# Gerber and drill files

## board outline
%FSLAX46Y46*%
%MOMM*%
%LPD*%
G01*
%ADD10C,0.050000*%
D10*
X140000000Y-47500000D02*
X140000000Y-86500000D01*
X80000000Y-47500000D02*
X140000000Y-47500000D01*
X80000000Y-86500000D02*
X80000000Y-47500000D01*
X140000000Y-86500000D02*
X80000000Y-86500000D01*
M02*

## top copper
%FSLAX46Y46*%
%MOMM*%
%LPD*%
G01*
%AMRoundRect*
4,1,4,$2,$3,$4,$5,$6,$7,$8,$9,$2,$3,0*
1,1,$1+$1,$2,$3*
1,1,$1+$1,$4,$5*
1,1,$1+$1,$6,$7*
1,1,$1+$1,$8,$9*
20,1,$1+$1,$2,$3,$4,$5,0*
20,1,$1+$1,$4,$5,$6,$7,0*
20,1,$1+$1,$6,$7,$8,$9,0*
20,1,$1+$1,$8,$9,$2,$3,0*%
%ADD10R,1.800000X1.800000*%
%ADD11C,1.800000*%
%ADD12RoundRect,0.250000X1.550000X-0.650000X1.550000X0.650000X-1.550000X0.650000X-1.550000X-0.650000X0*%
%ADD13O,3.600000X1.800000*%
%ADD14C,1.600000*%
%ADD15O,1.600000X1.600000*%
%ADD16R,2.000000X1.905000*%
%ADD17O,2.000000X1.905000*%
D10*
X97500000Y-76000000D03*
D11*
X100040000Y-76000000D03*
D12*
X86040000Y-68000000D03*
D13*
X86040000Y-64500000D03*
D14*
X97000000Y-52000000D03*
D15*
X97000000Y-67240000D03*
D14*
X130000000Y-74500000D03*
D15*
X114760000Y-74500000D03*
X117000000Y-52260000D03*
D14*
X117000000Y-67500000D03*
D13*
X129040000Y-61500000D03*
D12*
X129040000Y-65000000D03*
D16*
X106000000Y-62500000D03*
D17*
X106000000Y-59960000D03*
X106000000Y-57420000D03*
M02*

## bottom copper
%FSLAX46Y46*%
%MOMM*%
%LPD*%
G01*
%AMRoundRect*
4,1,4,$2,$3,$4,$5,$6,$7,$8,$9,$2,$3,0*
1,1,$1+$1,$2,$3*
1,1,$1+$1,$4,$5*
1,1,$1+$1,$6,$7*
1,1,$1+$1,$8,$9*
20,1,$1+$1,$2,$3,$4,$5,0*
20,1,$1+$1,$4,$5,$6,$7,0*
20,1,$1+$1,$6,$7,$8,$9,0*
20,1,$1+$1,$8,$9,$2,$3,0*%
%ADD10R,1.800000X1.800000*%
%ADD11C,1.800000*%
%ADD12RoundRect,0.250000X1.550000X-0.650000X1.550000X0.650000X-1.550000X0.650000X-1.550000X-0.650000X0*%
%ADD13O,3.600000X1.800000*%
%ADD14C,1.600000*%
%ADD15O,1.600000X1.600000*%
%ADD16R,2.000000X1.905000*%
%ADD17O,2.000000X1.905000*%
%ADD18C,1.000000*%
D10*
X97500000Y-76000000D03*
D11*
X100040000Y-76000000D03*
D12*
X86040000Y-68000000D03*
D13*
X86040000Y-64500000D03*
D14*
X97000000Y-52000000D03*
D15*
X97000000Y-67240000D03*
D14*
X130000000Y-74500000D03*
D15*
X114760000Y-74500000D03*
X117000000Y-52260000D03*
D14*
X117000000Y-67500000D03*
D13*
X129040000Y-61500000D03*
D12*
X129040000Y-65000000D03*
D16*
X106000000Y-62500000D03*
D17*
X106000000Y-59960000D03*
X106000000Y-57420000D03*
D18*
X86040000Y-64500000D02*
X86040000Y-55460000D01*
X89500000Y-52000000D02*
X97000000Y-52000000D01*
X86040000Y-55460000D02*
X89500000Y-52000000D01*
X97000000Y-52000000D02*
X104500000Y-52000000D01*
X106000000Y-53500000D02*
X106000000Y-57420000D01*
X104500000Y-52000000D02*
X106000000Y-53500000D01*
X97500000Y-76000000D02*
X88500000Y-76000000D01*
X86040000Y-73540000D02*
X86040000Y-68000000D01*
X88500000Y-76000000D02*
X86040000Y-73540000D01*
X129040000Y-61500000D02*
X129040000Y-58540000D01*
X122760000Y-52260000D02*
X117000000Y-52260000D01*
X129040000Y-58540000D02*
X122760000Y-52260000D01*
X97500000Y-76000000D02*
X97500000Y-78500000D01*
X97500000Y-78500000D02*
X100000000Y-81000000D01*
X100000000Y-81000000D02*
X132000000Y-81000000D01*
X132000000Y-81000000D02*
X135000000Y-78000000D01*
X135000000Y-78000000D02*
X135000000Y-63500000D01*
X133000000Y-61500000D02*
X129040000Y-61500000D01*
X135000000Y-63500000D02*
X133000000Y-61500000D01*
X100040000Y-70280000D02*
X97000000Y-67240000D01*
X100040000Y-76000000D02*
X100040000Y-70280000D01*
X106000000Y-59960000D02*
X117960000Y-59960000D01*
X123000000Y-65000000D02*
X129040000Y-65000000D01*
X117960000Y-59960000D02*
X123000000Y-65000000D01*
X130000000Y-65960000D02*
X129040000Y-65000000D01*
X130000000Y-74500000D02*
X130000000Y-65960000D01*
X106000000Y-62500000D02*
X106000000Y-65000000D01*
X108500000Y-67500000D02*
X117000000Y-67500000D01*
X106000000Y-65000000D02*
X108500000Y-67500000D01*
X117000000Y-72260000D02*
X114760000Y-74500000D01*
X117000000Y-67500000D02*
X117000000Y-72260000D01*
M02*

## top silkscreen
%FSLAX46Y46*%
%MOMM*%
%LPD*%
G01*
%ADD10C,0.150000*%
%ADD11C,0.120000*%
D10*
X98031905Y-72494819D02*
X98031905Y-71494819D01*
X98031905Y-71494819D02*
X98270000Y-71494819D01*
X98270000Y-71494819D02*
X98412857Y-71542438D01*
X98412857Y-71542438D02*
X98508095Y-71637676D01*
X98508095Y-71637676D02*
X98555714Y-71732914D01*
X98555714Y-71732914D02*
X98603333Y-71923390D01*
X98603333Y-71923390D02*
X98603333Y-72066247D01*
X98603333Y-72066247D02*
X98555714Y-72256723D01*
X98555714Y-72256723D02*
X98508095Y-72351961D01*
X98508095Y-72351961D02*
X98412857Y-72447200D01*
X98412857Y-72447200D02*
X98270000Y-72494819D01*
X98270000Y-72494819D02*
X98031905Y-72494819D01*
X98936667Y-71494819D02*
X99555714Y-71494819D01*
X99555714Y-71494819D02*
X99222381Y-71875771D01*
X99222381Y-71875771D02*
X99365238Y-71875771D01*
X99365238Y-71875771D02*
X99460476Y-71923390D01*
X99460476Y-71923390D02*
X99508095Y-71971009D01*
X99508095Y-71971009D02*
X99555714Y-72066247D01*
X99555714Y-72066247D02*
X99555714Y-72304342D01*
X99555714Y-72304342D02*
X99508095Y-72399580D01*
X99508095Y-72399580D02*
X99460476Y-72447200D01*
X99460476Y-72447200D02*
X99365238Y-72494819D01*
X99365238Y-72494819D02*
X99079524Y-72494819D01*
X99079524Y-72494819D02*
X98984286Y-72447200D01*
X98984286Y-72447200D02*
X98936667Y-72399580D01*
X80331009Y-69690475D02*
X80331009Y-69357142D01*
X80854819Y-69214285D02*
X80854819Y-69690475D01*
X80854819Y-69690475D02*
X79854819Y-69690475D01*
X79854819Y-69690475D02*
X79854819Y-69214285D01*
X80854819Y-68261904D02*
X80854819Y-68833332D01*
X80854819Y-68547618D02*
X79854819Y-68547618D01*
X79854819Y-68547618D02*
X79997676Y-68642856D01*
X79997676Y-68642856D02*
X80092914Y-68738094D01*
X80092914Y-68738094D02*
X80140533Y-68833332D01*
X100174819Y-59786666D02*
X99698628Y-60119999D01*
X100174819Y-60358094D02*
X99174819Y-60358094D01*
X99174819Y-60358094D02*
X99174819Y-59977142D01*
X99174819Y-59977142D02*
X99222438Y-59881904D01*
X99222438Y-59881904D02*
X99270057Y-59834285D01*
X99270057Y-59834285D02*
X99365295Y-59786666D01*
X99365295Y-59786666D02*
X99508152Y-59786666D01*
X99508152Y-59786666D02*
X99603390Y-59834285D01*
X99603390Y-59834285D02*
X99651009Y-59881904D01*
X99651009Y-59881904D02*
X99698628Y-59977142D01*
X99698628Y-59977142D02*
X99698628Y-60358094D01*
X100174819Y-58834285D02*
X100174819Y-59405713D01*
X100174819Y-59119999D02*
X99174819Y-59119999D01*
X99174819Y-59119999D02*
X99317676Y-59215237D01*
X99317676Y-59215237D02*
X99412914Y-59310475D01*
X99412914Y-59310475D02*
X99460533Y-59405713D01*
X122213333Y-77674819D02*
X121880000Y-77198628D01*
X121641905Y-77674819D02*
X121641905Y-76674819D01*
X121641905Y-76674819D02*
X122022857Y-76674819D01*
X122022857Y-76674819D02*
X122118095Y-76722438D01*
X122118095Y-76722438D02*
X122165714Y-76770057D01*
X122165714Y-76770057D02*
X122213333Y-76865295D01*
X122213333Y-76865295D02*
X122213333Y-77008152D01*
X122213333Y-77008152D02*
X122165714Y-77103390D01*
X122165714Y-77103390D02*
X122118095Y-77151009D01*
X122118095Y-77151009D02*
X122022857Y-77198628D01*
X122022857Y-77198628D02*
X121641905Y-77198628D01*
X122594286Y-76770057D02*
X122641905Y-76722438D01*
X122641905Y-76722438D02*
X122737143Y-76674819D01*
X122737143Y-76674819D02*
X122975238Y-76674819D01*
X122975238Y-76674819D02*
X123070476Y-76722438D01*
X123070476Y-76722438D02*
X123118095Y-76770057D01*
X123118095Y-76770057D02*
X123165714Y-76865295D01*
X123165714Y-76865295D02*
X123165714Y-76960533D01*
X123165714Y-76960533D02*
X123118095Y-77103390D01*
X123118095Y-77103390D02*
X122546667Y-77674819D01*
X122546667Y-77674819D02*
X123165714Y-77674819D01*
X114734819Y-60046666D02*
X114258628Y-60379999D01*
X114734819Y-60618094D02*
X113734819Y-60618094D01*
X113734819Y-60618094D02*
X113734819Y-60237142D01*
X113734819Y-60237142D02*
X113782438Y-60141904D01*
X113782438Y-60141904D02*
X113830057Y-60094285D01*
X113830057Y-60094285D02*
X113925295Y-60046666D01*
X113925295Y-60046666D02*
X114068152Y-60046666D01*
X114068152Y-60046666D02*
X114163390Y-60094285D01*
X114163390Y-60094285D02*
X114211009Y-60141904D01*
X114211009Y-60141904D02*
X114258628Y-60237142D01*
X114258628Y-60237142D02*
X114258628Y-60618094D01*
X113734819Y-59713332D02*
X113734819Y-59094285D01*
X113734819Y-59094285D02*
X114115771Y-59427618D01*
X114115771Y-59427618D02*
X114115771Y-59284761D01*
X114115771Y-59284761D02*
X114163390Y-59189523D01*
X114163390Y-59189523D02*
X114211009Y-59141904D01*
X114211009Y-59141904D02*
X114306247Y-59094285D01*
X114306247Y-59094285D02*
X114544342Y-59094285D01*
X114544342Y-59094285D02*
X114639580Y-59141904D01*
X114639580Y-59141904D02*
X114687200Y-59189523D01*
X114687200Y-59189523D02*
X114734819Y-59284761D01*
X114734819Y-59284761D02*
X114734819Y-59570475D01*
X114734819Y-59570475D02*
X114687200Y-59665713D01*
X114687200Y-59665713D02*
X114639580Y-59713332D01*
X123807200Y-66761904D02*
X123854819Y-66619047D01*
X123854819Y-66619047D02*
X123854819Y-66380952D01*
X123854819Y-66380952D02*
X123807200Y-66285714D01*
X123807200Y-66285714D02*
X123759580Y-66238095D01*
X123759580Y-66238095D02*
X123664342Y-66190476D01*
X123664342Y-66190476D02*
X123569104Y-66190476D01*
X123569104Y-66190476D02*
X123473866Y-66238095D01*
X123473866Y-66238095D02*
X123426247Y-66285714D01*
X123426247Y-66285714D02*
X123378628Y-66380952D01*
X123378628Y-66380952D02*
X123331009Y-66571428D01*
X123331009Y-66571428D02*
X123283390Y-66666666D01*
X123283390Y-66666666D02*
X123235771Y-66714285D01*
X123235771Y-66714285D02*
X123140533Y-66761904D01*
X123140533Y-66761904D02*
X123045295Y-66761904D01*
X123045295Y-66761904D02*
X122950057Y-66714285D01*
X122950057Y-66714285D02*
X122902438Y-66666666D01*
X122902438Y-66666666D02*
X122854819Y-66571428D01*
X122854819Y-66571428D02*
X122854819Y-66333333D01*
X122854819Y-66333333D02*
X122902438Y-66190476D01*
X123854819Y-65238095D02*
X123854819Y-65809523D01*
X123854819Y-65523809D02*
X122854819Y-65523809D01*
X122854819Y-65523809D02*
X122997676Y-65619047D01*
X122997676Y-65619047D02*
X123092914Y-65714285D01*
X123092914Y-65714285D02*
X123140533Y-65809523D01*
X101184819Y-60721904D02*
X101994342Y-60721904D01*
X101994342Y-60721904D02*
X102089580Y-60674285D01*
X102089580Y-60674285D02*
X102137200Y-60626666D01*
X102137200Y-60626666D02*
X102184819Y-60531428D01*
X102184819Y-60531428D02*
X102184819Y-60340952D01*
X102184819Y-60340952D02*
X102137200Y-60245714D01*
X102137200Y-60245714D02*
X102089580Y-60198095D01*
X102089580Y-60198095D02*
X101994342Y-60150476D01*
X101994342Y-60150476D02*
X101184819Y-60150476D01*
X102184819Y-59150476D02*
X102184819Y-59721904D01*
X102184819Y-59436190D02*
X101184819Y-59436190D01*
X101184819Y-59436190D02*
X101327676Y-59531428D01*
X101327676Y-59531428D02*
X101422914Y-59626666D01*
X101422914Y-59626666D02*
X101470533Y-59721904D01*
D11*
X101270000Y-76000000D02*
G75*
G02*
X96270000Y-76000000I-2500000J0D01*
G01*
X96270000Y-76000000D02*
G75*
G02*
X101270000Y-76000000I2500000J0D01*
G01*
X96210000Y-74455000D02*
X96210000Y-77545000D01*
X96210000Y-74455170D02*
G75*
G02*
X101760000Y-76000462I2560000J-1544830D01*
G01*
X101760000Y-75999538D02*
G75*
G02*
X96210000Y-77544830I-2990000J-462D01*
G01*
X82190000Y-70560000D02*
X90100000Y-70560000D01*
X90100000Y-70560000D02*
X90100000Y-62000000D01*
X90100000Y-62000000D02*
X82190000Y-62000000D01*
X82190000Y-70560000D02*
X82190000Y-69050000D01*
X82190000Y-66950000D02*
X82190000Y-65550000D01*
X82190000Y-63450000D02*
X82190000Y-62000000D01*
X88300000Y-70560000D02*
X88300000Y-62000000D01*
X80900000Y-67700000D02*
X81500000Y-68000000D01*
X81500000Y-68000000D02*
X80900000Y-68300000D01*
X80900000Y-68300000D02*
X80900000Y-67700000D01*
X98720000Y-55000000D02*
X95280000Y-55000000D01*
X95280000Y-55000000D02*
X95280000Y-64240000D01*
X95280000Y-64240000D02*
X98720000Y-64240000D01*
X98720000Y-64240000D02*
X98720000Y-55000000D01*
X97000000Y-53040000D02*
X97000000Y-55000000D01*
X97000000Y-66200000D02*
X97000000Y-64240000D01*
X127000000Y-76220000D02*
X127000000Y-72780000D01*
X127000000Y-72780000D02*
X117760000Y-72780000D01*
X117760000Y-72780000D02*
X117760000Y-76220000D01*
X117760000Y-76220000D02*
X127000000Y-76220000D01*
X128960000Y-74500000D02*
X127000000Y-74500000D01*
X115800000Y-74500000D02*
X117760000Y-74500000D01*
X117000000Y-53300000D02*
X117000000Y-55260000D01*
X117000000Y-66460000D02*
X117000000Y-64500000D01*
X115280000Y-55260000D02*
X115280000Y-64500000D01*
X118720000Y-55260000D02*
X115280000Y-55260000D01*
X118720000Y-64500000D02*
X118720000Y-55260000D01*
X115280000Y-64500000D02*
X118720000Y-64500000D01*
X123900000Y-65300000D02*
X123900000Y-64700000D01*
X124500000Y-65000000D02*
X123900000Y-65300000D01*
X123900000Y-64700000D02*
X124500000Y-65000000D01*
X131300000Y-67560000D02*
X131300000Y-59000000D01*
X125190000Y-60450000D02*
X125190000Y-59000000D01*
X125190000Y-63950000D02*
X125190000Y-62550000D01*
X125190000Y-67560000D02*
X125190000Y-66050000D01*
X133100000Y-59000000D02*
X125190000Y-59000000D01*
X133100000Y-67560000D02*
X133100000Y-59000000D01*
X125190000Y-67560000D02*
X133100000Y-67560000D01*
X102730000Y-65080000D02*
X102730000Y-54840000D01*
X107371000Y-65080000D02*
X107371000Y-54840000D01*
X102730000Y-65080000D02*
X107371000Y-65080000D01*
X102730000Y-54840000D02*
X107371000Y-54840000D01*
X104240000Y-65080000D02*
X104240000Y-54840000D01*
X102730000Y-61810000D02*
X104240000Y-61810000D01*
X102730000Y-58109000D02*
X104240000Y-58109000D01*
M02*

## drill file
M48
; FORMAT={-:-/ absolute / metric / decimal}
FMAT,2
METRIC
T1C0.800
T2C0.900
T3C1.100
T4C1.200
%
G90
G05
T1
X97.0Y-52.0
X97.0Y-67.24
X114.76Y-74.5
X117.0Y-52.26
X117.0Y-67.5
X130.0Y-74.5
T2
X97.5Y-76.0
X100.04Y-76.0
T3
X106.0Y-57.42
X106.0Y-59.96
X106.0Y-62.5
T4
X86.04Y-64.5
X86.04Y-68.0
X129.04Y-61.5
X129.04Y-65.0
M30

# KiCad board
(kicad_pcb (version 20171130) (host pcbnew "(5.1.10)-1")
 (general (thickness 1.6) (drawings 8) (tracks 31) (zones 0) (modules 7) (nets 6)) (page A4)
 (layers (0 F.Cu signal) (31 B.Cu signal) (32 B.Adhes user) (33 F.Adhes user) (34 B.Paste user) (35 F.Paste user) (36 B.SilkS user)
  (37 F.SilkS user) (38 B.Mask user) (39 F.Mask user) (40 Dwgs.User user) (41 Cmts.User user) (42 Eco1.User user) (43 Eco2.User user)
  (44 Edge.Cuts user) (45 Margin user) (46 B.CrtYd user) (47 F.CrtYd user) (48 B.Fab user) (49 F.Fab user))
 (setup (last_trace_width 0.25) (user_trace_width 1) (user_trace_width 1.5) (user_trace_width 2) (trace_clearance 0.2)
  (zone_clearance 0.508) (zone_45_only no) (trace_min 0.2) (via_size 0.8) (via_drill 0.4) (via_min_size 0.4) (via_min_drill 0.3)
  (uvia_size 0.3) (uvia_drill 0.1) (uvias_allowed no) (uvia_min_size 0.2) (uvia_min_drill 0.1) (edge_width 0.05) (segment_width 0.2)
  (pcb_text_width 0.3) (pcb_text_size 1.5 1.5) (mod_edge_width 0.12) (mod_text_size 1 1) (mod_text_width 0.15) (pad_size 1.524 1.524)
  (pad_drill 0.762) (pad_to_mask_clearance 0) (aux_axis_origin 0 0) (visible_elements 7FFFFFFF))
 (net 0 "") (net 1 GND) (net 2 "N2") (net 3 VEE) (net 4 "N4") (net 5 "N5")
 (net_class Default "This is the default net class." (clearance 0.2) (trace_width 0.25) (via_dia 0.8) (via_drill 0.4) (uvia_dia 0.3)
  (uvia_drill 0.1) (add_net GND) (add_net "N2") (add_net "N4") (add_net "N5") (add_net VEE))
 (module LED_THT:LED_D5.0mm (layer F.Cu) (at 97.5 76)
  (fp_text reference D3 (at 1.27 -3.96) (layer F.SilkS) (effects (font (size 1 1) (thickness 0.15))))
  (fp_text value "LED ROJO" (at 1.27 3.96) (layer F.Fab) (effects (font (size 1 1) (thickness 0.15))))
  (fp_circle (center 1.27 0) (end 3.77 0) (layer F.SilkS) (width 0.12))
  (fp_line (start -1.29 -1.545) (end -1.29 1.545) (layer F.SilkS) (width 0.12))
  (fp_arc (start 1.27 0) (end -1.29 -1.54483) (angle 148.9) (layer F.SilkS) (width 0.12))
  (fp_arc (start 1.27 0) (end -1.29 1.54483) (angle -148.9) (layer F.SilkS) (width 0.12))
  (pad 1 thru_hole rect (at 0 0) (size 1.8 1.8) (drill 0.9) (layers *.Cu *.Mask) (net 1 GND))
  (pad 2 thru_hole circle (at 2.54 0) (size 1.8 1.8) (drill 0.9) (layers *.Cu *.Mask) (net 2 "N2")))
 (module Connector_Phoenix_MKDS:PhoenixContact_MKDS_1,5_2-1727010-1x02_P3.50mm (layer F.Cu) (at 83.5 68 90)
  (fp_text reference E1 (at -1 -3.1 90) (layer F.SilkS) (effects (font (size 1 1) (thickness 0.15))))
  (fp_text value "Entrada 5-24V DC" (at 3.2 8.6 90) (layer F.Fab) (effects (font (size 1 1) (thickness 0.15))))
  (fp_line (start -2.56 -1.31) (end -2.56 6.6) (layer F.SilkS) (width 0.12))
  (fp_line (start -2.56 6.6) (end 6 6.6) (layer F.SilkS) (width 0.12))
  (fp_line (start 6 6.6) (end 6 -1.31) (layer F.SilkS) (width 0.12))
  (fp_line (start -2.56 -1.31) (end -1.05 -1.31) (layer F.SilkS) (width 0.12))
  (fp_line (start 1.05 -1.31) (end 2.45 -1.31) (layer F.SilkS) (width 0.12))
  (fp_line (start 4.55 -1.31) (end 6 -1.31) (layer F.SilkS) (width 0.12))
  (fp_line (start -2.56 4.8) (end 6 4.8) (layer F.SilkS) (width 0.12))
  (fp_line (start 0.3 -2.6) (end 0 -2) (layer F.SilkS) (width 0.12))
  (fp_line (start 0 -2) (end -0.3 -2.6) (layer F.SilkS) (width 0.12))
  (fp_line (start -0.3 -2.6) (end 0.3 -2.6) (layer F.SilkS) (width 0.12))
  (pad 1 thru_hole roundrect (at 0 2.54 90) (size 1.8 3.6) (drill 1.2) (layers *.Cu *.Mask) (roundrect_rratio 0.1388888888888889)
   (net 1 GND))
  (pad 2 thru_hole oval (at 3.5 2.54 90) (size 1.8 3.6) (drill 1.2) (layers *.Cu *.Mask) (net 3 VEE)))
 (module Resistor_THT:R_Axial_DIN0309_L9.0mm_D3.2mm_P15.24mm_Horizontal (layer F.Cu) (at 97 52 270)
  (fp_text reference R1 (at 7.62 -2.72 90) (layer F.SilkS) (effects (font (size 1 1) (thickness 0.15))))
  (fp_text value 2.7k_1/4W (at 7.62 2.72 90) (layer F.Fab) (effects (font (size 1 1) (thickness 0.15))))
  (fp_line (start 3 -1.72) (end 3 1.72) (layer F.SilkS) (width 0.12))
  (fp_line (start 3 1.72) (end 12.24 1.72) (layer F.SilkS) (width 0.12))
  (fp_line (start 12.24 1.72) (end 12.24 -1.72) (layer F.SilkS) (width 0.12))
  (fp_line (start 12.24 -1.72) (end 3 -1.72) (layer F.SilkS) (width 0.12))
  (fp_line (start 1.04 0) (end 3 0) (layer F.SilkS) (width 0.12))
  (fp_line (start 14.2 0) (end 12.24 0) (layer F.SilkS) (width 0.12))
  (pad 1 thru_hole circle (at 0 0 270) (size 1.6 1.6) (drill 0.8) (layers *.Cu *.Mask) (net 3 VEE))
  (pad 2 thru_hole oval (at 15.24 0 270) (size 1.6 1.6) (drill 0.8) (layers *.Cu *.Mask) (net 2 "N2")))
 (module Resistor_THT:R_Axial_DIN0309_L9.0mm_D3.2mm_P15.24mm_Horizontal (layer F.Cu) (at 130 74.5 180)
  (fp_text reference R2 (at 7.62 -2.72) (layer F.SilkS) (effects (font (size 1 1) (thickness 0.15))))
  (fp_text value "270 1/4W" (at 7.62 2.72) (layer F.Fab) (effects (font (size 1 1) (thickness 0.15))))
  (fp_line (start 3 -1.72) (end 3 1.72) (layer F.SilkS) (width 0.12))
  (fp_line (start 3 1.72) (end 12.24 1.72) (layer F.SilkS) (width 0.12))
  (fp_line (start 12.24 1.72) (end 12.24 -1.72) (layer F.SilkS) (width 0.12))
  (fp_line (start 12.24 -1.72) (end 3 -1.72) (layer F.SilkS) (width 0.12))
  (fp_line (start 1.04 0) (end 3 0) (layer F.SilkS) (width 0.12))
  (fp_line (start 14.2 0) (end 12.24 0) (layer F.SilkS) (width 0.12))
  (pad 1 thru_hole circle (at 0 0 180) (size 1.6 1.6) (drill 0.8) (layers *.Cu *.Mask) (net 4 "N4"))
  (pad 2 thru_hole oval (at 15.24 0 180) (size 1.6 1.6) (drill 0.8) (layers *.Cu *.Mask) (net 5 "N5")))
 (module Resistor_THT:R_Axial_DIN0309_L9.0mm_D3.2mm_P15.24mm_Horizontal (layer F.Cu) (at 117 67.5 90)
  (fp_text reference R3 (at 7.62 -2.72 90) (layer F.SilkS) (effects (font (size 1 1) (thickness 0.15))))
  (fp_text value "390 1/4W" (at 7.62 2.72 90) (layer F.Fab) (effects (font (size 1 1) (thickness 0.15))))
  (fp_line (start 14.2 0) (end 12.24 0) (layer F.SilkS) (width 0.12))
  (fp_line (start 1.04 0) (end 3 0) (layer F.SilkS) (width 0.12))
  (fp_line (start 12.24 -1.72) (end 3 -1.72) (layer F.SilkS) (width 0.12))
  (fp_line (start 12.24 1.72) (end 12.24 -1.72) (layer F.SilkS) (width 0.12))
  (fp_line (start 3 1.72) (end 12.24 1.72) (layer F.SilkS) (width 0.12))
  (fp_line (start 3 -1.72) (end 3 1.72) (layer F.SilkS) (width 0.12))
  (pad 2 thru_hole oval (at 15.24 0 90) (size 1.6 1.6) (drill 0.8) (layers *.Cu *.Mask) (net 1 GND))
  (pad 1 thru_hole circle (at 0 0 90) (size 1.6 1.6) (drill 0.8) (layers *.Cu *.Mask) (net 5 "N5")))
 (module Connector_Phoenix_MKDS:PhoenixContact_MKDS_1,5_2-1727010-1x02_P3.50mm (layer F.Cu) (at 126.5 65 90)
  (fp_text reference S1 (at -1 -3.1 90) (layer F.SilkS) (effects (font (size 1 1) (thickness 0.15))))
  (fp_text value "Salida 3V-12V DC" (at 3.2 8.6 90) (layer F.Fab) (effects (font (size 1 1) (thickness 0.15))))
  (fp_line (start -0.3 -2.6) (end 0.3 -2.6) (layer F.SilkS) (width 0.12))
  (fp_line (start 0 -2) (end -0.3 -2.6) (layer F.SilkS) (width 0.12))
  (fp_line (start 0.3 -2.6) (end 0 -2) (layer F.SilkS) (width 0.12))
  (fp_line (start -2.56 4.8) (end 6 4.8) (layer F.SilkS) (width 0.12))
  (fp_line (start 4.55 -1.31) (end 6 -1.31) (layer F.SilkS) (width 0.12))
  (fp_line (start 1.05 -1.31) (end 2.45 -1.31) (layer F.SilkS) (width 0.12))
  (fp_line (start -2.56 -1.31) (end -1.05 -1.31) (layer F.SilkS) (width 0.12))
  (fp_line (start 6 6.6) (end 6 -1.31) (layer F.SilkS) (width 0.12))
  (fp_line (start -2.56 6.6) (end 6 6.6) (layer F.SilkS) (width 0.12))
  (fp_line (start -2.56 -1.31) (end -2.56 6.6) (layer F.SilkS) (width 0.12))
  (pad 2 thru_hole oval (at 3.5 2.54 90) (size 1.8 3.6) (drill 1.2) (layers *.Cu *.Mask) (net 1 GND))
  (pad 1 thru_hole roundrect (at 0 2.54 90) (size 1.8 3.6) (drill 1.2) (layers *.Cu *.Mask) (roundrect_rratio 0.1388888888888889)
   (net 4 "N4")))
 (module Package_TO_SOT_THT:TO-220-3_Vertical (layer F.Cu) (at 106 62.5 90)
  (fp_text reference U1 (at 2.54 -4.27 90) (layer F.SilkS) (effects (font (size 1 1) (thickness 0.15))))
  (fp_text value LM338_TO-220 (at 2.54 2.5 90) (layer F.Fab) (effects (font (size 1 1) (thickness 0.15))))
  (fp_line (start -2.58 -3.27) (end 7.66 -3.27) (layer F.SilkS) (width 0.12))
  (fp_line (start -2.58 1.371) (end 7.66 1.371) (layer F.SilkS) (width 0.12))
  (fp_line (start -2.58 -3.27) (end -2.58 1.371) (layer F.SilkS) (width 0.12))
  (fp_line (start 7.66 -3.27) (end 7.66 1.371) (layer F.SilkS) (width 0.12))
  (fp_line (start -2.58 -1.76) (end 7.66 -1.76) (layer F.SilkS) (width 0.12))
  (fp_line (start 0.69 -3.27) (end 0.69 -1.76) (layer F.SilkS) (width 0.12))
  (fp_line (start 4.391 -3.27) (end 4.391 -1.76) (layer F.SilkS) (width 0.12))
  (pad 1 thru_hole rect (at 0 0 90) (size 1.905 2) (drill 1.1) (layers *.Cu *.Mask) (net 5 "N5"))
  (pad 2 thru_hole oval (at 2.54 0 90) (size 1.905 2) (drill 1.1) (layers *.Cu *.Mask) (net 4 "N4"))
  (pad 3 thru_hole oval (at 5.08 0 90) (size 1.905 2) (drill 1.1) (layers *.Cu *.Mask) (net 3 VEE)))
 (gr_line (start 140 47.5) (end 140 86.5) (layer Edge.Cuts) (width 0.05))
 (gr_line (start 80 47.5) (end 140 47.5) (layer Edge.Cuts) (width 0.05))
 (gr_line (start 80 86.5) (end 80 47.5) (layer Edge.Cuts) (width 0.05))
 (gr_line (start 140 86.5) (end 80 86.5) (layer Edge.Cuts) (width 0.05))
 (segment (start 86.04 64.5) (end 86.04 55.46) (width 1) (layer B.Cu) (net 3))
 (segment (start 89.5 52) (end 97 52) (width 1) (layer B.Cu) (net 3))
 (segment (start 86.04 55.46) (end 89.5 52) (width 1) (layer B.Cu) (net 3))
 (segment (start 97 52) (end 104.5 52) (width 1) (layer B.Cu) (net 3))
 (segment (start 106 53.5) (end 106 57.42) (width 1) (layer B.Cu) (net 3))
 (segment (start 104.5 52) (end 106 53.5) (width 1) (layer B.Cu) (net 3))
 (segment (start 97.5 76) (end 88.5 76) (width 1) (layer B.Cu) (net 1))
 (segment (start 86.04 73.54) (end 86.04 68) (width 1) (layer B.Cu) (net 1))
 (segment (start 88.5 76) (end 86.04 73.54) (width 1) (layer B.Cu) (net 1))
 (segment (start 129.04 61.5) (end 129.04 58.54) (width 1) (layer B.Cu) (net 1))
 (segment (start 122.76 52.26) (end 117 52.26) (width 1) (layer B.Cu) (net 1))
 (segment (start 129.04 58.54) (end 122.76 52.26) (width 1) (layer B.Cu) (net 1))
 (segment (start 97.5 76) (end 97.5 78.5) (width 1) (layer B.Cu) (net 1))
 (segment (start 97.5 78.5) (end 100 81) (width 1) (layer B.Cu) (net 1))
 (segment (start 100 81) (end 132 81) (width 1) (layer B.Cu) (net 1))
 (segment (start 132 81) (end 135 78) (width 1) (layer B.Cu) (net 1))
 (segment (start 135 78) (end 135 63.5) (width 1) (layer B.Cu) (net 1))
 (segment (start 133 61.5) (end 129.04 61.5) (width 1) (layer B.Cu) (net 1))
 (segment (start 135 63.5) (end 133 61.5) (width 1) (layer B.Cu) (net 1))
 (segment (start 100.04 70.28) (end 97 67.24) (width 1) (layer B.Cu) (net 2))
 (segment (start 100.04 76) (end 100.04 70.28) (width 1) (layer B.Cu) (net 2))
 (segment (start 106 59.96) (end 117.96 59.96) (width 1) (layer B.Cu) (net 4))
 (segment (start 123 65) (end 129.04 65) (width 1) (layer B.Cu) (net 4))
 (segment (start 117.96 59.96) (end 123 65) (width 1) (layer B.Cu) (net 4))
 (segment (start 130 65.96) (end 129.04 65) (width 1) (layer B.Cu) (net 4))
 (segment (start 130 74.5) (end 130 65.96) (width 1) (layer B.Cu) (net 4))
 (segment (start 106 62.5) (end 106 65) (width 1) (layer B.Cu) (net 5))
 (segment (start 108.5 67.5) (end 117 67.5) (width 1) (layer B.Cu) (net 5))
 (segment (start 106 65) (end 108.5 67.5) (width 1) (layer B.Cu) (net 5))
 (segment (start 117 72.26) (end 114.76 74.5) (width 1) (layer B.Cu) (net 5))
 (segment (start 117 67.5) (end 117 72.26) (width 1) (layer B.Cu) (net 5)))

